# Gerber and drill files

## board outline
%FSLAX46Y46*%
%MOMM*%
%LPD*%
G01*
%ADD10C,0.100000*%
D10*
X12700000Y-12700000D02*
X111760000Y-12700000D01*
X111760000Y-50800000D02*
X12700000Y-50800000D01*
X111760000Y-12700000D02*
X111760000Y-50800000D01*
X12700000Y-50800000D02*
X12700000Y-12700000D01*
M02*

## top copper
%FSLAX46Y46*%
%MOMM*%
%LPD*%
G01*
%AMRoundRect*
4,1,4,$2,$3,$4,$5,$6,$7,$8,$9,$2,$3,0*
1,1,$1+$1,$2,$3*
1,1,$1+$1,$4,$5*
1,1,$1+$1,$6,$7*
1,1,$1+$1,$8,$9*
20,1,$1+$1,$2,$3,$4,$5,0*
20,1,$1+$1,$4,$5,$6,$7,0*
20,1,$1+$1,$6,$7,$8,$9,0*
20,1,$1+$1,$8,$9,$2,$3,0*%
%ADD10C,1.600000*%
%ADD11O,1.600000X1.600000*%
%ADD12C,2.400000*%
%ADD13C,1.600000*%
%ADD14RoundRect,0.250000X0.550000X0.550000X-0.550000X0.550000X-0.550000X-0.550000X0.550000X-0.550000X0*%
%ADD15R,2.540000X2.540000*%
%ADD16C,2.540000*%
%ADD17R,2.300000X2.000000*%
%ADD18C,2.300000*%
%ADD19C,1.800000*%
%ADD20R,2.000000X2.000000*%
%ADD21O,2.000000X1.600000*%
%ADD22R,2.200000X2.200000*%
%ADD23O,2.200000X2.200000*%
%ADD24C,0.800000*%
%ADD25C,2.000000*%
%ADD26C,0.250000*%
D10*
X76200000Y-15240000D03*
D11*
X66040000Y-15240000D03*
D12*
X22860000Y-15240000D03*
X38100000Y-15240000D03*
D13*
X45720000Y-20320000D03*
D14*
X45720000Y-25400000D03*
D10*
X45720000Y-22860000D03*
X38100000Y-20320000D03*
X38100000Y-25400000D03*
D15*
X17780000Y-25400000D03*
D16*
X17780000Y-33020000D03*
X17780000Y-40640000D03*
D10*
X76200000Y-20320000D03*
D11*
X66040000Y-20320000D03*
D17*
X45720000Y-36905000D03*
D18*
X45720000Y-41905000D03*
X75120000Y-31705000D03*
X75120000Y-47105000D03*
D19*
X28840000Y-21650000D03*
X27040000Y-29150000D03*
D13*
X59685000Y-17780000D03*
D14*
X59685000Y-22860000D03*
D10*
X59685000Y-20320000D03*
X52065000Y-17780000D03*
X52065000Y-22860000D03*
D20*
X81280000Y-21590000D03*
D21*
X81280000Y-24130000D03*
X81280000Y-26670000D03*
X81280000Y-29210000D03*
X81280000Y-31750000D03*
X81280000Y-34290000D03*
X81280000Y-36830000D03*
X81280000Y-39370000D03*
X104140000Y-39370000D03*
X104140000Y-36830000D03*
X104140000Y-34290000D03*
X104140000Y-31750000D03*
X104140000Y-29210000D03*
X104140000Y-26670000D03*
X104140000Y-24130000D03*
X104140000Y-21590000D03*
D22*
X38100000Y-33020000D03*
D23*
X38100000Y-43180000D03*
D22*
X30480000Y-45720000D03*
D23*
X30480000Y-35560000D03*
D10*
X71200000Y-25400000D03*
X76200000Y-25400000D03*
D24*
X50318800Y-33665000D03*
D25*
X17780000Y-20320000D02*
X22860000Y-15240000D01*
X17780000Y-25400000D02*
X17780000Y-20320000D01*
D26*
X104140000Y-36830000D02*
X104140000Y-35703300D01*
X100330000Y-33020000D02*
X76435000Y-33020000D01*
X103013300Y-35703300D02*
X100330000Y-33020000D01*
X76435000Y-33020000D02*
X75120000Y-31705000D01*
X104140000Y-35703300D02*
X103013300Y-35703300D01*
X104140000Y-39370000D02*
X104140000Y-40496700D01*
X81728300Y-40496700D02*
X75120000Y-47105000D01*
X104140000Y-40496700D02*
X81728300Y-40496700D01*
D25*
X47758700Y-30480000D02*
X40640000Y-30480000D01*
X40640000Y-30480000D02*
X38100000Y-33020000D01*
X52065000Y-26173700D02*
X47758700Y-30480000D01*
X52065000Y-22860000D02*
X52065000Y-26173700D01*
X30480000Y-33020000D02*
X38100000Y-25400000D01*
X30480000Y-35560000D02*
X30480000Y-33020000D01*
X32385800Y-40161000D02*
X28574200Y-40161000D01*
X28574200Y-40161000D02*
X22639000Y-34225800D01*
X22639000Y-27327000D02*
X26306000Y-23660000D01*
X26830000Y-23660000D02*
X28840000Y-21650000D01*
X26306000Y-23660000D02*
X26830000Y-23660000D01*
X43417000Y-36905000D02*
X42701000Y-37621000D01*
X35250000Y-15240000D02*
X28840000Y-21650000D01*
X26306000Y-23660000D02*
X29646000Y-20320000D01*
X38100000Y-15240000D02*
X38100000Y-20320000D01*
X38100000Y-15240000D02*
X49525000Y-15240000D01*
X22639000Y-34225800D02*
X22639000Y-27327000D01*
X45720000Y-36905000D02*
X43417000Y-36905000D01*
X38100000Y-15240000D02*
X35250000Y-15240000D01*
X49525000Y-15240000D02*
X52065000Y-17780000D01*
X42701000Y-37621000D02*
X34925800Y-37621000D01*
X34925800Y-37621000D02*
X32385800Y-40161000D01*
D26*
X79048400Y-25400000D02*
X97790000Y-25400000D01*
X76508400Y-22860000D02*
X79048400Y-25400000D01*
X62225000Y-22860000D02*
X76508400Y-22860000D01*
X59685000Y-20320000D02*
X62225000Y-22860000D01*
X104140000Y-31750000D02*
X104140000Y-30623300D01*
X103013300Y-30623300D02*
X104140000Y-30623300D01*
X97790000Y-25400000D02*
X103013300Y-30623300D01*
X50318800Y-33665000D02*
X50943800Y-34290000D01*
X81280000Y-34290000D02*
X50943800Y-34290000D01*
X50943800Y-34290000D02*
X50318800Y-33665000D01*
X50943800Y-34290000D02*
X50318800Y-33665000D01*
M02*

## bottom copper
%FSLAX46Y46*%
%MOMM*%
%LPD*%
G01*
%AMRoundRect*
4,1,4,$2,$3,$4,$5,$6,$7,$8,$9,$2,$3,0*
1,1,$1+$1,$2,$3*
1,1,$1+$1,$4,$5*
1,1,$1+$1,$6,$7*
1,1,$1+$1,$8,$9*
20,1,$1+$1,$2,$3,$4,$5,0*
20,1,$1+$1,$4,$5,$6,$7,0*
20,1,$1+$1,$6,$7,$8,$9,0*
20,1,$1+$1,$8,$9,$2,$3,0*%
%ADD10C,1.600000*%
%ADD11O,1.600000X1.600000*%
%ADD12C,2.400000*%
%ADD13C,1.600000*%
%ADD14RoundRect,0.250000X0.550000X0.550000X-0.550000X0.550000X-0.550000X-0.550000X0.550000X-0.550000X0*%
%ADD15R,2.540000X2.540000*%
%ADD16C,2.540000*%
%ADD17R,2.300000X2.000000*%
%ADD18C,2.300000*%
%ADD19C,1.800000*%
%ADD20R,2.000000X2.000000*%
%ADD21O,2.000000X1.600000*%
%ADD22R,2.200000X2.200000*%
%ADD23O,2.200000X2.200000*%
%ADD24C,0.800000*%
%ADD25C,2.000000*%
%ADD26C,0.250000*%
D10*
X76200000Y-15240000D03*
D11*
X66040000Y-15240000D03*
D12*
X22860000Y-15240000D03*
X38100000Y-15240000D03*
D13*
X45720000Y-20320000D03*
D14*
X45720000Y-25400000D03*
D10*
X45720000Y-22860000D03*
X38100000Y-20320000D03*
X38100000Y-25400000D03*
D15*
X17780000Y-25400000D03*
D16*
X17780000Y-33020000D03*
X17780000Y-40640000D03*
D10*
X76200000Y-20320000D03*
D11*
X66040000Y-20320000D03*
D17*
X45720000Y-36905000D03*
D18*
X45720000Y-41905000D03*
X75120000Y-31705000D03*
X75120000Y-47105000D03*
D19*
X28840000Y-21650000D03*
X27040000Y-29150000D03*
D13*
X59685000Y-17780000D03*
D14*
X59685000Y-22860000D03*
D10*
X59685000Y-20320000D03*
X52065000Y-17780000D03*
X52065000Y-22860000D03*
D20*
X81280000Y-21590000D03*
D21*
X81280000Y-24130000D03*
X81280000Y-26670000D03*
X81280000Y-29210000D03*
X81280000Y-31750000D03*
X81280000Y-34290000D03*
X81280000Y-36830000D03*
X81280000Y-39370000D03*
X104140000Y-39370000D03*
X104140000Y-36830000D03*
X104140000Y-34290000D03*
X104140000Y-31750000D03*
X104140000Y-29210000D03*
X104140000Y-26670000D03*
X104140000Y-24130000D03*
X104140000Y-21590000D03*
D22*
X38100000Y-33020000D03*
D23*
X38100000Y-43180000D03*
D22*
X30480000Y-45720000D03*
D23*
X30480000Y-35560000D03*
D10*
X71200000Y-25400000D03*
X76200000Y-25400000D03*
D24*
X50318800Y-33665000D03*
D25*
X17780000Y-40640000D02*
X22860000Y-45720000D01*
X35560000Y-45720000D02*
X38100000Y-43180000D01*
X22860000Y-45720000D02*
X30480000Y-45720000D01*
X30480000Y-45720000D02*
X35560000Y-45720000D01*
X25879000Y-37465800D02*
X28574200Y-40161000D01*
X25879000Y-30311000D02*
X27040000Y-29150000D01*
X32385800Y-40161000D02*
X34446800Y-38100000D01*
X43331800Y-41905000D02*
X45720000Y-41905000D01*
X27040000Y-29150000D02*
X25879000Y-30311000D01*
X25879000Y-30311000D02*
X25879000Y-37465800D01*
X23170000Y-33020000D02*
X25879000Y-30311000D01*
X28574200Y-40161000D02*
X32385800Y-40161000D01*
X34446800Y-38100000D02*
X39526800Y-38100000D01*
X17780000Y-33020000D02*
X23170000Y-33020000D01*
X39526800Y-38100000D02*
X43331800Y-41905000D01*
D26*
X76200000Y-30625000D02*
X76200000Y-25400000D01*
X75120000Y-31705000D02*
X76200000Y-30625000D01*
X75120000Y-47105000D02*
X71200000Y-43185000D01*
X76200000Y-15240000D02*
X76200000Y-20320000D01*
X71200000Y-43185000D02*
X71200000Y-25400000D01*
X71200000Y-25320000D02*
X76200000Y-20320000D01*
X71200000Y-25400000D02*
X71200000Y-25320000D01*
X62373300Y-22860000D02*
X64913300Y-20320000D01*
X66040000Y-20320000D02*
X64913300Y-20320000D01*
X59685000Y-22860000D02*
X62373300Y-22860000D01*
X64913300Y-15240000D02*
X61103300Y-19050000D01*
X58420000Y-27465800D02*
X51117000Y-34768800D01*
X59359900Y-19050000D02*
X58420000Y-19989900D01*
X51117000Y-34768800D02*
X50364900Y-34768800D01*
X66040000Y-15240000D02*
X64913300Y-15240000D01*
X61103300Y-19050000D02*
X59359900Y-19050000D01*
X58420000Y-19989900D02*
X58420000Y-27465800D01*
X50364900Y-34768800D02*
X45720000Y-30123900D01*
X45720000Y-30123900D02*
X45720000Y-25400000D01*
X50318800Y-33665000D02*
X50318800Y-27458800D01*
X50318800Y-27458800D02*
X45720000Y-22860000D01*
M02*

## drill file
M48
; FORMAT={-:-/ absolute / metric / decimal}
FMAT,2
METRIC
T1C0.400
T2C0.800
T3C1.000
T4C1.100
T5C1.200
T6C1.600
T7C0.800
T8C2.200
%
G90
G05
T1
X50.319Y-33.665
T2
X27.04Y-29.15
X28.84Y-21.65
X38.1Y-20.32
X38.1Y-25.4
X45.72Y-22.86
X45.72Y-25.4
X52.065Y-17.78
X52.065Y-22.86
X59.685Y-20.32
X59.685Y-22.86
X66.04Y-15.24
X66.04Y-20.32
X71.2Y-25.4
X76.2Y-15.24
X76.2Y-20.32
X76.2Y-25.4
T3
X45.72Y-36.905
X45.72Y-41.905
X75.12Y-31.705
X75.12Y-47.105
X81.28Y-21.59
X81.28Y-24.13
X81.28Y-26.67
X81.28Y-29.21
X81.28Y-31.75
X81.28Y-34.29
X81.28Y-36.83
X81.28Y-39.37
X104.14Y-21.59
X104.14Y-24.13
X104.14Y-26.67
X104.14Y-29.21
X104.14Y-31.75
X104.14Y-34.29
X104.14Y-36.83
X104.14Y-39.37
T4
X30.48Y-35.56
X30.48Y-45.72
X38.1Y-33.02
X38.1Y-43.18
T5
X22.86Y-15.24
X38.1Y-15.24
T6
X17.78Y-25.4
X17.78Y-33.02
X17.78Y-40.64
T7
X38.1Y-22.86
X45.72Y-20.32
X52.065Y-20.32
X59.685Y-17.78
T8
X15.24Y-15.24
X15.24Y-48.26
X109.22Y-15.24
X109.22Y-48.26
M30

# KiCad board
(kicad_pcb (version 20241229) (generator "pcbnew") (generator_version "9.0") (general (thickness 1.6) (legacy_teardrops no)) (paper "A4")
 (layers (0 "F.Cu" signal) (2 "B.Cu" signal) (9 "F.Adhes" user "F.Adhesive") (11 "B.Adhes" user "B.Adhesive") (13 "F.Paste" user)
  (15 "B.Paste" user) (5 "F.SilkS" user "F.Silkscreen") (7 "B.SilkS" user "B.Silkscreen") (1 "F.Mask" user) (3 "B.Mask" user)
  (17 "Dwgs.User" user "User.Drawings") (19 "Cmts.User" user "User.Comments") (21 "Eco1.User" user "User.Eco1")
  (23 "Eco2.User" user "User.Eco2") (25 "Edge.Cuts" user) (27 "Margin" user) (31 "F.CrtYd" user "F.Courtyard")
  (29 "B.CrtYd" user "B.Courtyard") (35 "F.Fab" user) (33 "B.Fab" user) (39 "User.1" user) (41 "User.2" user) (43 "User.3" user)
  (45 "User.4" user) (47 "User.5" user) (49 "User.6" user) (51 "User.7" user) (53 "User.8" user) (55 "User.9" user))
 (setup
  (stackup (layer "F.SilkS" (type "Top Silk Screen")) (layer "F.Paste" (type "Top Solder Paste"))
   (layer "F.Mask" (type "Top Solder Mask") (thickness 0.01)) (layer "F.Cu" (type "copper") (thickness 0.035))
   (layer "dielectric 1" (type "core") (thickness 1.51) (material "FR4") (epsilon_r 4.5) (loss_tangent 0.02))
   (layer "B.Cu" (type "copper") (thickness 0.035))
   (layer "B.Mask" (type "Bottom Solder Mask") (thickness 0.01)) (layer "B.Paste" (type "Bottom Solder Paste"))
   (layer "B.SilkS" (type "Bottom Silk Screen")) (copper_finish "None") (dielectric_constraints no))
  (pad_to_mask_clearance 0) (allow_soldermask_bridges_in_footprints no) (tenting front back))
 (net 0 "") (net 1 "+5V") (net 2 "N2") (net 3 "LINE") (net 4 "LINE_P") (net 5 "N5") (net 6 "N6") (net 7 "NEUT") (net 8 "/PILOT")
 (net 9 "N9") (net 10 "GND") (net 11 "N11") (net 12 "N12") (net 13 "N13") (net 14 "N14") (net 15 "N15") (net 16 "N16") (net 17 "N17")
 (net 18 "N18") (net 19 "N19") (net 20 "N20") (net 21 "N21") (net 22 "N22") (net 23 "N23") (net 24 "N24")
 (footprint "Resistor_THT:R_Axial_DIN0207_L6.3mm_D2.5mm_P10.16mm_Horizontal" (layer "F.Cu") (at 76.2 15.24 180)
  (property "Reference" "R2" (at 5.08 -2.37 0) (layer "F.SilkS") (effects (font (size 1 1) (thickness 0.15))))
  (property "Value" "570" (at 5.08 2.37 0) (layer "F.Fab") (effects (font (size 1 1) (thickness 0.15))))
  (pad "1" thru_hole circle (at 0 0 180) (size 1.6 1.6) (drill 0.8) (layers "*.Cu" "*.Mask") (remove_unused_layers no) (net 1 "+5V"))
  (pad "2" thru_hole oval (at 10.16 0 180) (size 1.6 1.6) (drill 0.8) (layers "*.Cu" "*.Mask") (remove_unused_layers no) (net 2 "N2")))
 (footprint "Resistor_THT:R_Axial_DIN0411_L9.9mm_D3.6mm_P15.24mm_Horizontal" (layer "F.Cu") (at 22.86 15.24)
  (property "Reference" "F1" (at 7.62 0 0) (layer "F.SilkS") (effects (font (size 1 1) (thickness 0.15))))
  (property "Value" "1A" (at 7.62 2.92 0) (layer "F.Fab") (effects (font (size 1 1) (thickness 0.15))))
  (pad "1" thru_hole circle (at 0 0) (size 2.4 2.4) (drill 1.2) (layers "*.Cu" "*.Mask") (remove_unused_layers no) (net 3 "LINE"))
  (pad "2" thru_hole circle (at 15.24 0) (size 2.4 2.4) (drill 1.2) (layers "*.Cu" "*.Mask") (remove_unused_layers no) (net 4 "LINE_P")))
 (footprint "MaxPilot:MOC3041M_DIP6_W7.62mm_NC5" (layer "F.Cu") (at 45.72 25.4 180)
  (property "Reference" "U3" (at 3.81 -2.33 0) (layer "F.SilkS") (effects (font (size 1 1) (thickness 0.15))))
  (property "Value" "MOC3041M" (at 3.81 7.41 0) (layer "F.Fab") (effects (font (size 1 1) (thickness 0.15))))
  (pad "" np_thru_hole circle (at 0 5.08 180) (size 1.6 1.6) (drill 0.8) (layers "*.Cu" "*.Mask"))
  (pad "" np_thru_hole circle (at 7.62 2.54 180) (size 0.8 0.8) (drill 0.8) (layers "*.Cu" "*.Mask"))
  (pad "1" thru_hole roundrect (at 0 0 180) (size 1.6 1.6) (drill 0.8) (layers "*.Cu" "*.Mask") (remove_unused_layers no)
   (roundrect_rratio 0.15625) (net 2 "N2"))
  (pad "2" thru_hole circle (at 0 2.54 180) (size 1.6 1.6) (drill 0.8) (layers "*.Cu" "*.Mask") (remove_unused_layers no) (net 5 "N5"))
  (pad "4" thru_hole circle (at 7.62 5.08 180) (size 1.6 1.6) (drill 0.8) (layers "*.Cu" "*.Mask") (remove_unused_layers no)
   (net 4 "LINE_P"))
  (pad "6" thru_hole circle (at 7.62 0 180) (size 1.6 1.6) (drill 0.8) (layers "*.Cu" "*.Mask") (remove_unused_layers no) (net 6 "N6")))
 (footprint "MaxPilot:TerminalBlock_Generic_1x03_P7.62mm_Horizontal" (layer "F.Cu") (at 17.78 25.4 -90)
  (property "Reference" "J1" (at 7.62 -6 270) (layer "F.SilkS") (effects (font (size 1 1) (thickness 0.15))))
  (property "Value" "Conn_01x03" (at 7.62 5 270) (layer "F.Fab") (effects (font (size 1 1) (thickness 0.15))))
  (pad "1" thru_hole rect (at 0 0 270) (size 2.54 2.54) (drill 1.6) (layers "*.Cu" "*.Mask") (remove_unused_layers no) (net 3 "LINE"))
  (pad "2" thru_hole circle (at 7.62 0 270) (size 2.54 2.54) (drill 1.6) (layers "*.Cu" "*.Mask") (remove_unused_layers no) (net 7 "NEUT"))
  (pad "3" thru_hole circle (at 15.24 0 270) (size 2.54 2.54) (drill 1.6) (layers "*.Cu" "*.Mask") (remove_unused_layers no)
   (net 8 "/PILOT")))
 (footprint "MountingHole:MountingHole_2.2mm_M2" (layer "F.Cu") (at 15.24 15.24)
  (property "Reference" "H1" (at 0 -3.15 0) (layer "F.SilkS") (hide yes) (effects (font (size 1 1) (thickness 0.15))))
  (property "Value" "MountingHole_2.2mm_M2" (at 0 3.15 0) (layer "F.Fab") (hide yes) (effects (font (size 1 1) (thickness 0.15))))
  (pad "" np_thru_hole circle (at 0 0) (size 2.2 2.2) (drill 2.2) (layers "*.Cu" "*.Mask")))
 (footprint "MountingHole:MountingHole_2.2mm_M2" (layer "F.Cu") (at 109.22 48.26)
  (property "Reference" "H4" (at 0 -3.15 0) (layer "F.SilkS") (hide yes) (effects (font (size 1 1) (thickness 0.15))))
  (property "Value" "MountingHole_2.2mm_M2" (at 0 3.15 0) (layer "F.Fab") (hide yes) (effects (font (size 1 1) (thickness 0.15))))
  (pad "" np_thru_hole circle (at 0 0) (size 2.2 2.2) (drill 2.2) (layers "*.Cu" "*.Mask")))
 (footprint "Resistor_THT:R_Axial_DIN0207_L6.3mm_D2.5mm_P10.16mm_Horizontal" (layer "F.Cu") (at 76.2 20.32 180)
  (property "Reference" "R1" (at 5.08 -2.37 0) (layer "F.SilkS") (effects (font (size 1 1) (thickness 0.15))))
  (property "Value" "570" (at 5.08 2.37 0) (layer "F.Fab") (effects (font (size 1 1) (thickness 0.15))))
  (pad "1" thru_hole circle (at 0 0 180) (size 1.6 1.6) (drill 0.8) (layers "*.Cu" "*.Mask") (remove_unused_layers no) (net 1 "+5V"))
  (pad "2" thru_hole oval (at 10.16 0 180) (size 1.6 1.6) (drill 0.8) (layers "*.Cu" "*.Mask") (remove_unused_layers no) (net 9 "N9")))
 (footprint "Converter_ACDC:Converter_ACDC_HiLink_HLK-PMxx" (layer "F.Cu") (at 45.72 36.905)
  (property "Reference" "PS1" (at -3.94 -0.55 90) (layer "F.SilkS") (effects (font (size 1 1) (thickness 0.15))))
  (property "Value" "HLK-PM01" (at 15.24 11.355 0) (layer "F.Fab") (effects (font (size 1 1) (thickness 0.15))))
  (pad "1" thru_hole rect (at 0 0) (size 2.3 2) (drill 1) (layers "*.Cu" "*.Mask") (remove_unused_layers no) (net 4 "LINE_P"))
  (pad "2" thru_hole circle (at 0 5) (size 2.3 2.3) (drill 1) (layers "*.Cu" "*.Mask") (remove_unused_layers no) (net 7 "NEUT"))
  (pad "3" thru_hole circle (at 29.4 -5.2) (size 2.3 2.3) (drill 1) (layers "*.Cu" "*.Mask") (remove_unused_layers no) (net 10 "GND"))
  (pad "4" thru_hole circle (at 29.4 10.2) (size 2.3 2.3) (drill 1) (layers "*.Cu" "*.Mask") (remove_unused_layers no) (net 1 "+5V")))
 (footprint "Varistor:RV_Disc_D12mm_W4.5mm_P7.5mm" (layer "F.Cu") (at 28.84 21.65 -90)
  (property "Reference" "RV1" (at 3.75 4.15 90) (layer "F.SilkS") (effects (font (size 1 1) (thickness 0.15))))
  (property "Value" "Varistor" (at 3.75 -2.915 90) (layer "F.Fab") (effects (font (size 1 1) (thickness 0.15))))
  (pad "1" thru_hole circle (at 0 0 270) (size 1.8 1.8) (drill 0.8) (layers "*.Cu" "*.Mask") (remove_unused_layers no) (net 4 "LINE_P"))
  (pad "2" thru_hole circle (at 7.5 1.8 270) (size 1.8 1.8) (drill 0.8) (layers "*.Cu" "*.Mask") (remove_unused_layers no) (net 7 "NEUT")))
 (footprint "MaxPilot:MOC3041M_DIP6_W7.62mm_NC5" (layer "F.Cu") (at 59.685 22.86 180)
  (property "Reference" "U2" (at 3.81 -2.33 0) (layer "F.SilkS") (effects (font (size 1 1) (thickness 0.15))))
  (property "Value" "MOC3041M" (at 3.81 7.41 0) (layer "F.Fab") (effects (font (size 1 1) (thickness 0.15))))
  (pad "" np_thru_hole circle (at 0 5.08 180) (size 1.6 1.6) (drill 0.8) (layers "*.Cu" "*.Mask"))
  (pad "" np_thru_hole circle (at 7.62 2.54 180) (size 0.8 0.8) (drill 0.8) (layers "*.Cu" "*.Mask"))
  (pad "1" thru_hole roundrect (at 0 0 180) (size 1.6 1.6) (drill 0.8) (layers "*.Cu" "*.Mask") (remove_unused_layers no)
   (roundrect_rratio 0.15625) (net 9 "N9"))
  (pad "2" thru_hole circle (at 0 2.54 180) (size 1.6 1.6) (drill 0.8) (layers "*.Cu" "*.Mask") (remove_unused_layers no) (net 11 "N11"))
  (pad "4" thru_hole circle (at 7.62 5.08 180) (size 1.6 1.6) (drill 0.8) (layers "*.Cu" "*.Mask") (remove_unused_layers no)
   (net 4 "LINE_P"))
  (pad "6" thru_hole circle (at 7.62 0 180) (size 1.6 1.6) (drill 0.8) (layers "*.Cu" "*.Mask") (remove_unused_layers no) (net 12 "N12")))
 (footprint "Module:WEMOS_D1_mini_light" (layer "F.Cu") (at 81.28 21.59)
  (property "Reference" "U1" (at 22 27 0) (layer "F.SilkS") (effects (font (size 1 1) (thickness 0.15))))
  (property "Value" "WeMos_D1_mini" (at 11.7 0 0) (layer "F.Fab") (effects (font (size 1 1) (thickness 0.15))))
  (pad "1" thru_hole rect (at 0 0) (size 2 2) (drill 1) (layers "*.Cu" "*.Mask") (remove_unused_layers no) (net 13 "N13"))
  (pad "2" thru_hole oval (at 0 2.54) (size 2 1.6) (drill 1) (layers "*.Cu" "*.Mask") (remove_unused_layers no) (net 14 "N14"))
  (pad "3" thru_hole oval (at 0 5.08) (size 2 1.6) (drill 1) (layers "*.Cu" "*.Mask") (remove_unused_layers no) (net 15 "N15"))
  (pad "4" thru_hole oval (at 0 7.62) (size 2 1.6) (drill 1) (layers "*.Cu" "*.Mask") (remove_unused_layers no) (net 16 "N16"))
  (pad "5" thru_hole oval (at 0 10.16) (size 2 1.6) (drill 1) (layers "*.Cu" "*.Mask") (remove_unused_layers no) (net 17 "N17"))
  (pad "6" thru_hole oval (at 0 12.7) (size 2 1.6) (drill 1) (layers "*.Cu" "*.Mask") (remove_unused_layers no) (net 5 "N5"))
  (pad "7" thru_hole oval (at 0 15.24) (size 2 1.6) (drill 1) (layers "*.Cu" "*.Mask") (remove_unused_layers no) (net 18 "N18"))
  (pad "8" thru_hole oval (at 0 17.78) (size 2 1.6) (drill 1) (layers "*.Cu" "*.Mask") (remove_unused_layers no) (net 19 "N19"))
  (pad "9" thru_hole oval (at 22.86 17.78) (size 2 1.6) (drill 1) (layers "*.Cu" "*.Mask") (remove_unused_layers no) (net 1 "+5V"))
  (pad "10" thru_hole oval (at 22.86 15.24) (size 2 1.6) (drill 1) (layers "*.Cu" "*.Mask") (remove_unused_layers no) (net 10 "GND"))
  (pad "11" thru_hole oval (at 22.86 12.7) (size 2 1.6) (drill 1) (layers "*.Cu" "*.Mask") (remove_unused_layers no) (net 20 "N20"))
  (pad "12" thru_hole oval (at 22.86 10.16) (size 2 1.6) (drill 1) (layers "*.Cu" "*.Mask") (remove_unused_layers no) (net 11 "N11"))
  (pad "13" thru_hole oval (at 22.86 7.62) (size 2 1.6) (drill 1) (layers "*.Cu" "*.Mask") (remove_unused_layers no) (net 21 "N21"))
  (pad "14" thru_hole oval (at 22.86 5.08) (size 2 1.6) (drill 1) (layers "*.Cu" "*.Mask") (remove_unused_layers no) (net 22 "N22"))
  (pad "15" thru_hole oval (at 22.86 2.54) (size 2 1.6) (drill 1) (layers "*.Cu" "*.Mask") (remove_unused_layers no) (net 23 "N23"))
  (pad "16" thru_hole oval (at 22.86 0) (size 2 1.6) (drill 1) (layers "*.Cu" "*.Mask") (remove_unused_layers no) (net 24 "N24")))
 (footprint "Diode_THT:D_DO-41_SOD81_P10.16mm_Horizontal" (layer "F.Cu") (at 38.1 33.02 -90)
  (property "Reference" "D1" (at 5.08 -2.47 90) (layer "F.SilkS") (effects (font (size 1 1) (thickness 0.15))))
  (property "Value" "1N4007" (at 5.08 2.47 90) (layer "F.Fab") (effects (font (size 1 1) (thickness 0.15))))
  (pad "1" thru_hole rect (at 0 0 270) (size 2.2 2.2) (drill 1.1) (layers "*.Cu" "*.Mask") (remove_unused_layers no) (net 12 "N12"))
  (pad "2" thru_hole oval (at 10.16 0 270) (size 2.2 2.2) (drill 1.1) (layers "*.Cu" "*.Mask") (remove_unused_layers no) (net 8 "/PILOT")))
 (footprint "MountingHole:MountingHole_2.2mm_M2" (layer "F.Cu") (at 15.24 48.26)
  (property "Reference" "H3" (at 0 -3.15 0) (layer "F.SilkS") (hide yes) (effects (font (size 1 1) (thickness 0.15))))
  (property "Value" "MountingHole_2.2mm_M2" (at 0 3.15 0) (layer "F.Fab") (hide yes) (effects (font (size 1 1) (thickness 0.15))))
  (pad "" np_thru_hole circle (at 0 0) (size 2.2 2.2) (drill 2.2) (layers "*.Cu" "*.Mask")))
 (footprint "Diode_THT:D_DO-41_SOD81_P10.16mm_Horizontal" (layer "F.Cu") (at 30.48 45.72 90)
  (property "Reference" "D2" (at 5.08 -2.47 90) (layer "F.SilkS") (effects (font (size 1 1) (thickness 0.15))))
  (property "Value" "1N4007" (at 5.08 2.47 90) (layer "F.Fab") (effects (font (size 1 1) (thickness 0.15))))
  (pad "1" thru_hole rect (at 0 0 90) (size 2.2 2.2) (drill 1.1) (layers "*.Cu" "*.Mask") (remove_unused_layers no) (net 8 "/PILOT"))
  (pad "2" thru_hole oval (at 10.16 0 90) (size 2.2 2.2) (drill 1.1) (layers "*.Cu" "*.Mask") (remove_unused_layers no) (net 6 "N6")))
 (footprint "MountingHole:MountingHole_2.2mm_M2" (layer "F.Cu") (at 109.22 15.24)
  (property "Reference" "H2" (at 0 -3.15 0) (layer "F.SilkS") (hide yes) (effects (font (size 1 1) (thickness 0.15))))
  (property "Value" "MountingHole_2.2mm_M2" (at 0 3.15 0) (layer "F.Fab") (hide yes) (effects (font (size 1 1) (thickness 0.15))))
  (pad "" np_thru_hole circle (at 0 0) (size 2.2 2.2) (drill 2.2) (layers "*.Cu" "*.Mask")))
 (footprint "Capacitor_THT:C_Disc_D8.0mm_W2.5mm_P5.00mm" (layer "F.Cu") (at 71.2 25.4)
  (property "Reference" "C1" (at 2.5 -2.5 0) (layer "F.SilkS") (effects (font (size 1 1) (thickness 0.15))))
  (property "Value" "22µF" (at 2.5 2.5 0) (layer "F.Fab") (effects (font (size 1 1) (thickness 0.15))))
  (pad "1" thru_hole circle (at 0 0) (size 1.6 1.6) (drill 0.8) (layers "*.Cu" "*.Mask") (remove_unused_layers no) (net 1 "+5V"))
  (pad "2" thru_hole circle (at 5 0) (size 1.6 1.6) (drill 0.8) (layers "*.Cu" "*.Mask") (remove_unused_layers no) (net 10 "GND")))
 (gr_line (start 12.7 12.7) (end 111.76 12.7) (stroke (width 0.1) (type solid)) (layer "Edge.Cuts"))
 (gr_line (start 111.76 50.8) (end 12.7 50.8) (stroke (width 0.1) (type solid)) (layer "Edge.Cuts"))
 (gr_line (start 111.76 12.7) (end 111.76 50.8) (stroke (width 0.1) (type solid)) (layer "Edge.Cuts"))
 (gr_line (start 12.7 50.8) (end 12.7 12.7) (stroke (width 0.1) (type solid)) (layer "Edge.Cuts"))
 (segment (start 17.78 40.64) (end 22.86 45.72) (width 2) (layer "B.Cu") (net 8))
 (segment (start 35.56 45.72) (end 38.1 43.18) (width 2) (layer "B.Cu") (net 8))
 (segment (start 22.86 45.72) (end 30.48 45.72) (width 2) (layer "B.Cu") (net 8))
 (segment (start 30.48 45.72) (end 35.56 45.72) (width 2) (layer "B.Cu") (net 8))
 (segment (start 17.78 20.32) (end 22.86 15.24) (width 2) (layer "F.Cu") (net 3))
 (segment (start 17.78 25.4) (end 17.78 20.32) (width 2) (layer "F.Cu") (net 3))
 (segment (start 25.879 37.4658) (end 28.5742 40.161) (width 2) (layer "B.Cu") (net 7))
 (segment (start 25.879 30.311) (end 27.04 29.15) (width 2) (layer "B.Cu") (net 7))
 (segment (start 32.3858 40.161) (end 34.4468 38.1) (width 2) (layer "B.Cu") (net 7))
 (segment (start 43.3318 41.905) (end 45.72 41.905) (width 2) (layer "B.Cu") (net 7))
 (segment (start 27.04 29.15) (end 25.879 30.311) (width 2) (layer "B.Cu") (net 7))
 (segment (start 25.879 30.311) (end 25.879 37.4658) (width 2) (layer "B.Cu") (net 7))
 (segment (start 23.17 33.02) (end 25.879 30.311) (width 2) (layer "B.Cu") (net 7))
 (segment (start 28.5742 40.161) (end 32.3858 40.161) (width 2) (layer "B.Cu") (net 7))
 (segment (start 34.4468 38.1) (end 39.5268 38.1) (width 2) (layer "B.Cu") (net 7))
 (segment (start 17.78 33.02) (end 23.17 33.02) (width 2) (layer "B.Cu") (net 7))
 (segment (start 39.5268 38.1) (end 43.3318 41.905) (width 2) (layer "B.Cu") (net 7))
 (segment (start 104.14 36.83) (end 104.14 35.7033) (width 0.25) (layer "F.Cu") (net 10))
 (segment (start 100.33 33.02) (end 76.435 33.02) (width 0.25) (layer "F.Cu") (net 10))
 (segment (start 103.0133 35.7033) (end 100.33 33.02) (width 0.25) (layer "F.Cu") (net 10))
 (segment (start 76.435 33.02) (end 75.12 31.705) (width 0.25) (layer "F.Cu") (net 10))
 (segment (start 104.14 35.7033) (end 103.0133 35.7033) (width 0.25) (layer "F.Cu") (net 10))
 (segment (start 76.2 30.625) (end 76.2 25.4) (width 0.25) (layer "B.Cu") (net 10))
 (segment (start 75.12 31.705) (end 76.2 30.625) (width 0.25) (layer "B.Cu") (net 10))
 (segment (start 104.14 39.37) (end 104.14 40.4967) (width 0.25) (layer "F.Cu") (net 1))
 (segment (start 81.7283 40.4967) (end 75.12 47.105) (width 0.25) (layer "F.Cu") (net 1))
 (segment (start 104.14 40.4967) (end 81.7283 40.4967) (width 0.25) (layer "F.Cu") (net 1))
 (segment (start 75.12 47.105) (end 71.2 43.185) (width 0.25) (layer "B.Cu") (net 1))
 (segment (start 76.2 15.24) (end 76.2 20.32) (width 0.25) (layer "B.Cu") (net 1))
 (segment (start 71.2 43.185) (end 71.2 25.4) (width 0.25) (layer "B.Cu") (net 1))
 (segment (start 71.2 25.32) (end 76.2 20.32) (width 0.25) (layer "B.Cu") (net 1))
 (segment (start 71.2 25.4) (end 71.2 25.32) (width 0.25) (layer "B.Cu") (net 1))
 (segment (start 62.3733 22.86) (end 64.9133 20.32) (width 0.25) (layer "B.Cu") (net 9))
 (segment (start 66.04 20.32) (end 64.9133 20.32) (width 0.25) (layer "B.Cu") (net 9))
 (segment (start 59.685 22.86) (end 62.3733 22.86) (width 0.25) (layer "B.Cu") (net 9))
 (segment (start 64.9133 15.24) (end 61.1033 19.05) (width 0.25) (layer "B.Cu") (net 2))
 (segment (start 58.42 27.4658) (end 51.117 34.7688) (width 0.25) (layer "B.Cu") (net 2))
 (segment (start 59.3599 19.05) (end 58.42 19.9899) (width 0.25) (layer "B.Cu") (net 2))
 (segment (start 51.117 34.7688) (end 50.3649 34.7688) (width 0.25) (layer "B.Cu") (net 2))
 (segment (start 66.04 15.24) (end 64.9133 15.24) (width 0.25) (layer "B.Cu") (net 2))
 (segment (start 61.1033 19.05) (end 59.3599 19.05) (width 0.25) (layer "B.Cu") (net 2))
 (segment (start 58.42 19.9899) (end 58.42 27.4658) (width 0.25) (layer "B.Cu") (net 2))
 (segment (start 50.3649 34.7688) (end 45.72 30.1239) (width 0.25) (layer "B.Cu") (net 2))
 (segment (start 45.72 30.1239) (end 45.72 25.4) (width 0.25) (layer "B.Cu") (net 2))
 (segment (start 47.7587 30.48) (end 40.64 30.48) (width 2) (layer "F.Cu") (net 12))
 (segment (start 40.64 30.48) (end 38.1 33.02) (width 2) (layer "F.Cu") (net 12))
 (segment (start 52.065 26.1737) (end 47.7587 30.48) (width 2) (layer "F.Cu") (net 12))
 (segment (start 52.065 22.86) (end 52.065 26.1737) (width 2) (layer "F.Cu") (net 12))
 (segment (start 30.48 33.02) (end 38.1 25.4) (width 2) (layer "F.Cu") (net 6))
 (segment (start 30.48 35.56) (end 30.48 33.02) (width 2) (layer "F.Cu") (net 6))
 (segment (start 32.3858 40.161) (end 28.5742 40.161) (width 2) (layer "F.Cu") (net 4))
 (segment (start 28.5742 40.161) (end 22.639 34.2258) (width 2) (layer "F.Cu") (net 4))
 (segment (start 22.639 27.327) (end 26.306 23.66) (width 2) (layer "F.Cu") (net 4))
 (segment (start 26.83 23.66) (end 28.84 21.65) (width 2) (layer "F.Cu") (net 4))
 (segment (start 26.306 23.66) (end 26.83 23.66) (width 2) (layer "F.Cu") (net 4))
 (segment (start 43.417 36.905) (end 42.701 37.621) (width 2) (layer "F.Cu") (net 4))
 (segment (start 35.25 15.24) (end 28.84 21.65) (width 2) (layer "F.Cu") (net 4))
 (segment (start 26.306 23.66) (end 29.646 20.32) (width 2) (layer "F.Cu") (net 4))
 (segment (start 38.1 15.24) (end 38.1 20.32) (width 2) (layer "F.Cu") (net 4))
 (segment (start 38.1 15.24) (end 49.525 15.24) (width 2) (layer "F.Cu") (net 4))
 (segment (start 22.639 34.2258) (end 22.639 27.327) (width 2) (layer "F.Cu") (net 4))
 (segment (start 45.72 36.905) (end 43.417 36.905) (width 2) (layer "F.Cu") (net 4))
 (segment (start 38.1 15.24) (end 35.25 15.24) (width 2) (layer "F.Cu") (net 4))
 (segment (start 49.525 15.24) (end 52.065 17.78) (width 2) (layer "F.Cu") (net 4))
 (segment (start 42.701 37.621) (end 34.9258 37.621) (width 2) (layer "F.Cu") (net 4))
 (segment (start 34.9258 37.621) (end 32.3858 40.161) (width 2) (layer "F.Cu") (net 4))
 (segment (start 79.0484 25.4) (end 97.79 25.4) (width 0.25) (layer "F.Cu") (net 11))
 (segment (start 76.5084 22.86) (end 79.0484 25.4) (width 0.25) (layer "F.Cu") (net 11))
 (segment (start 62.225 22.86) (end 76.5084 22.86) (width 0.25) (layer "F.Cu") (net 11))
 (segment (start 59.685 20.32) (end 62.225 22.86) (width 0.25) (layer "F.Cu") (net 11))
 (segment (start 104.14 31.75) (end 104.14 30.6233) (width 0.25) (layer "F.Cu") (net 11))
 (segment (start 103.0133 30.6233) (end 104.14 30.6233) (width 0.25) (layer "F.Cu") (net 11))
 (segment (start 97.79 25.4) (end 103.0133 30.6233) (width 0.25) (layer "F.Cu") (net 11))
 (segment (start 50.3188 33.665) (end 50.9438 34.29) (width 0.25) (layer "F.Cu") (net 5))
 (segment (start 81.28 34.29) (end 50.9438 34.29) (width 0.25) (layer "F.Cu") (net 5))
 (segment (start 50.9438 34.29) (end 50.3188 33.665) (width 0.25) (layer "F.Cu") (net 5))
 (segment (start 50.9438 34.29) (end 50.3188 33.665) (width 0.25) (layer "F.Cu") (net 5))
 (via (at 50.3188 33.665) (size 0.8) (drill 0.4) (layers "F.Cu" "B.Cu") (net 5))
 (segment (start 50.3188 33.665) (end 50.3188 27.4588) (width 0.25) (layer "B.Cu") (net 5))
 (segment (start 50.3188 27.4588) (end 45.72 22.86) (width 0.25) (layer "B.Cu") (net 5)))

